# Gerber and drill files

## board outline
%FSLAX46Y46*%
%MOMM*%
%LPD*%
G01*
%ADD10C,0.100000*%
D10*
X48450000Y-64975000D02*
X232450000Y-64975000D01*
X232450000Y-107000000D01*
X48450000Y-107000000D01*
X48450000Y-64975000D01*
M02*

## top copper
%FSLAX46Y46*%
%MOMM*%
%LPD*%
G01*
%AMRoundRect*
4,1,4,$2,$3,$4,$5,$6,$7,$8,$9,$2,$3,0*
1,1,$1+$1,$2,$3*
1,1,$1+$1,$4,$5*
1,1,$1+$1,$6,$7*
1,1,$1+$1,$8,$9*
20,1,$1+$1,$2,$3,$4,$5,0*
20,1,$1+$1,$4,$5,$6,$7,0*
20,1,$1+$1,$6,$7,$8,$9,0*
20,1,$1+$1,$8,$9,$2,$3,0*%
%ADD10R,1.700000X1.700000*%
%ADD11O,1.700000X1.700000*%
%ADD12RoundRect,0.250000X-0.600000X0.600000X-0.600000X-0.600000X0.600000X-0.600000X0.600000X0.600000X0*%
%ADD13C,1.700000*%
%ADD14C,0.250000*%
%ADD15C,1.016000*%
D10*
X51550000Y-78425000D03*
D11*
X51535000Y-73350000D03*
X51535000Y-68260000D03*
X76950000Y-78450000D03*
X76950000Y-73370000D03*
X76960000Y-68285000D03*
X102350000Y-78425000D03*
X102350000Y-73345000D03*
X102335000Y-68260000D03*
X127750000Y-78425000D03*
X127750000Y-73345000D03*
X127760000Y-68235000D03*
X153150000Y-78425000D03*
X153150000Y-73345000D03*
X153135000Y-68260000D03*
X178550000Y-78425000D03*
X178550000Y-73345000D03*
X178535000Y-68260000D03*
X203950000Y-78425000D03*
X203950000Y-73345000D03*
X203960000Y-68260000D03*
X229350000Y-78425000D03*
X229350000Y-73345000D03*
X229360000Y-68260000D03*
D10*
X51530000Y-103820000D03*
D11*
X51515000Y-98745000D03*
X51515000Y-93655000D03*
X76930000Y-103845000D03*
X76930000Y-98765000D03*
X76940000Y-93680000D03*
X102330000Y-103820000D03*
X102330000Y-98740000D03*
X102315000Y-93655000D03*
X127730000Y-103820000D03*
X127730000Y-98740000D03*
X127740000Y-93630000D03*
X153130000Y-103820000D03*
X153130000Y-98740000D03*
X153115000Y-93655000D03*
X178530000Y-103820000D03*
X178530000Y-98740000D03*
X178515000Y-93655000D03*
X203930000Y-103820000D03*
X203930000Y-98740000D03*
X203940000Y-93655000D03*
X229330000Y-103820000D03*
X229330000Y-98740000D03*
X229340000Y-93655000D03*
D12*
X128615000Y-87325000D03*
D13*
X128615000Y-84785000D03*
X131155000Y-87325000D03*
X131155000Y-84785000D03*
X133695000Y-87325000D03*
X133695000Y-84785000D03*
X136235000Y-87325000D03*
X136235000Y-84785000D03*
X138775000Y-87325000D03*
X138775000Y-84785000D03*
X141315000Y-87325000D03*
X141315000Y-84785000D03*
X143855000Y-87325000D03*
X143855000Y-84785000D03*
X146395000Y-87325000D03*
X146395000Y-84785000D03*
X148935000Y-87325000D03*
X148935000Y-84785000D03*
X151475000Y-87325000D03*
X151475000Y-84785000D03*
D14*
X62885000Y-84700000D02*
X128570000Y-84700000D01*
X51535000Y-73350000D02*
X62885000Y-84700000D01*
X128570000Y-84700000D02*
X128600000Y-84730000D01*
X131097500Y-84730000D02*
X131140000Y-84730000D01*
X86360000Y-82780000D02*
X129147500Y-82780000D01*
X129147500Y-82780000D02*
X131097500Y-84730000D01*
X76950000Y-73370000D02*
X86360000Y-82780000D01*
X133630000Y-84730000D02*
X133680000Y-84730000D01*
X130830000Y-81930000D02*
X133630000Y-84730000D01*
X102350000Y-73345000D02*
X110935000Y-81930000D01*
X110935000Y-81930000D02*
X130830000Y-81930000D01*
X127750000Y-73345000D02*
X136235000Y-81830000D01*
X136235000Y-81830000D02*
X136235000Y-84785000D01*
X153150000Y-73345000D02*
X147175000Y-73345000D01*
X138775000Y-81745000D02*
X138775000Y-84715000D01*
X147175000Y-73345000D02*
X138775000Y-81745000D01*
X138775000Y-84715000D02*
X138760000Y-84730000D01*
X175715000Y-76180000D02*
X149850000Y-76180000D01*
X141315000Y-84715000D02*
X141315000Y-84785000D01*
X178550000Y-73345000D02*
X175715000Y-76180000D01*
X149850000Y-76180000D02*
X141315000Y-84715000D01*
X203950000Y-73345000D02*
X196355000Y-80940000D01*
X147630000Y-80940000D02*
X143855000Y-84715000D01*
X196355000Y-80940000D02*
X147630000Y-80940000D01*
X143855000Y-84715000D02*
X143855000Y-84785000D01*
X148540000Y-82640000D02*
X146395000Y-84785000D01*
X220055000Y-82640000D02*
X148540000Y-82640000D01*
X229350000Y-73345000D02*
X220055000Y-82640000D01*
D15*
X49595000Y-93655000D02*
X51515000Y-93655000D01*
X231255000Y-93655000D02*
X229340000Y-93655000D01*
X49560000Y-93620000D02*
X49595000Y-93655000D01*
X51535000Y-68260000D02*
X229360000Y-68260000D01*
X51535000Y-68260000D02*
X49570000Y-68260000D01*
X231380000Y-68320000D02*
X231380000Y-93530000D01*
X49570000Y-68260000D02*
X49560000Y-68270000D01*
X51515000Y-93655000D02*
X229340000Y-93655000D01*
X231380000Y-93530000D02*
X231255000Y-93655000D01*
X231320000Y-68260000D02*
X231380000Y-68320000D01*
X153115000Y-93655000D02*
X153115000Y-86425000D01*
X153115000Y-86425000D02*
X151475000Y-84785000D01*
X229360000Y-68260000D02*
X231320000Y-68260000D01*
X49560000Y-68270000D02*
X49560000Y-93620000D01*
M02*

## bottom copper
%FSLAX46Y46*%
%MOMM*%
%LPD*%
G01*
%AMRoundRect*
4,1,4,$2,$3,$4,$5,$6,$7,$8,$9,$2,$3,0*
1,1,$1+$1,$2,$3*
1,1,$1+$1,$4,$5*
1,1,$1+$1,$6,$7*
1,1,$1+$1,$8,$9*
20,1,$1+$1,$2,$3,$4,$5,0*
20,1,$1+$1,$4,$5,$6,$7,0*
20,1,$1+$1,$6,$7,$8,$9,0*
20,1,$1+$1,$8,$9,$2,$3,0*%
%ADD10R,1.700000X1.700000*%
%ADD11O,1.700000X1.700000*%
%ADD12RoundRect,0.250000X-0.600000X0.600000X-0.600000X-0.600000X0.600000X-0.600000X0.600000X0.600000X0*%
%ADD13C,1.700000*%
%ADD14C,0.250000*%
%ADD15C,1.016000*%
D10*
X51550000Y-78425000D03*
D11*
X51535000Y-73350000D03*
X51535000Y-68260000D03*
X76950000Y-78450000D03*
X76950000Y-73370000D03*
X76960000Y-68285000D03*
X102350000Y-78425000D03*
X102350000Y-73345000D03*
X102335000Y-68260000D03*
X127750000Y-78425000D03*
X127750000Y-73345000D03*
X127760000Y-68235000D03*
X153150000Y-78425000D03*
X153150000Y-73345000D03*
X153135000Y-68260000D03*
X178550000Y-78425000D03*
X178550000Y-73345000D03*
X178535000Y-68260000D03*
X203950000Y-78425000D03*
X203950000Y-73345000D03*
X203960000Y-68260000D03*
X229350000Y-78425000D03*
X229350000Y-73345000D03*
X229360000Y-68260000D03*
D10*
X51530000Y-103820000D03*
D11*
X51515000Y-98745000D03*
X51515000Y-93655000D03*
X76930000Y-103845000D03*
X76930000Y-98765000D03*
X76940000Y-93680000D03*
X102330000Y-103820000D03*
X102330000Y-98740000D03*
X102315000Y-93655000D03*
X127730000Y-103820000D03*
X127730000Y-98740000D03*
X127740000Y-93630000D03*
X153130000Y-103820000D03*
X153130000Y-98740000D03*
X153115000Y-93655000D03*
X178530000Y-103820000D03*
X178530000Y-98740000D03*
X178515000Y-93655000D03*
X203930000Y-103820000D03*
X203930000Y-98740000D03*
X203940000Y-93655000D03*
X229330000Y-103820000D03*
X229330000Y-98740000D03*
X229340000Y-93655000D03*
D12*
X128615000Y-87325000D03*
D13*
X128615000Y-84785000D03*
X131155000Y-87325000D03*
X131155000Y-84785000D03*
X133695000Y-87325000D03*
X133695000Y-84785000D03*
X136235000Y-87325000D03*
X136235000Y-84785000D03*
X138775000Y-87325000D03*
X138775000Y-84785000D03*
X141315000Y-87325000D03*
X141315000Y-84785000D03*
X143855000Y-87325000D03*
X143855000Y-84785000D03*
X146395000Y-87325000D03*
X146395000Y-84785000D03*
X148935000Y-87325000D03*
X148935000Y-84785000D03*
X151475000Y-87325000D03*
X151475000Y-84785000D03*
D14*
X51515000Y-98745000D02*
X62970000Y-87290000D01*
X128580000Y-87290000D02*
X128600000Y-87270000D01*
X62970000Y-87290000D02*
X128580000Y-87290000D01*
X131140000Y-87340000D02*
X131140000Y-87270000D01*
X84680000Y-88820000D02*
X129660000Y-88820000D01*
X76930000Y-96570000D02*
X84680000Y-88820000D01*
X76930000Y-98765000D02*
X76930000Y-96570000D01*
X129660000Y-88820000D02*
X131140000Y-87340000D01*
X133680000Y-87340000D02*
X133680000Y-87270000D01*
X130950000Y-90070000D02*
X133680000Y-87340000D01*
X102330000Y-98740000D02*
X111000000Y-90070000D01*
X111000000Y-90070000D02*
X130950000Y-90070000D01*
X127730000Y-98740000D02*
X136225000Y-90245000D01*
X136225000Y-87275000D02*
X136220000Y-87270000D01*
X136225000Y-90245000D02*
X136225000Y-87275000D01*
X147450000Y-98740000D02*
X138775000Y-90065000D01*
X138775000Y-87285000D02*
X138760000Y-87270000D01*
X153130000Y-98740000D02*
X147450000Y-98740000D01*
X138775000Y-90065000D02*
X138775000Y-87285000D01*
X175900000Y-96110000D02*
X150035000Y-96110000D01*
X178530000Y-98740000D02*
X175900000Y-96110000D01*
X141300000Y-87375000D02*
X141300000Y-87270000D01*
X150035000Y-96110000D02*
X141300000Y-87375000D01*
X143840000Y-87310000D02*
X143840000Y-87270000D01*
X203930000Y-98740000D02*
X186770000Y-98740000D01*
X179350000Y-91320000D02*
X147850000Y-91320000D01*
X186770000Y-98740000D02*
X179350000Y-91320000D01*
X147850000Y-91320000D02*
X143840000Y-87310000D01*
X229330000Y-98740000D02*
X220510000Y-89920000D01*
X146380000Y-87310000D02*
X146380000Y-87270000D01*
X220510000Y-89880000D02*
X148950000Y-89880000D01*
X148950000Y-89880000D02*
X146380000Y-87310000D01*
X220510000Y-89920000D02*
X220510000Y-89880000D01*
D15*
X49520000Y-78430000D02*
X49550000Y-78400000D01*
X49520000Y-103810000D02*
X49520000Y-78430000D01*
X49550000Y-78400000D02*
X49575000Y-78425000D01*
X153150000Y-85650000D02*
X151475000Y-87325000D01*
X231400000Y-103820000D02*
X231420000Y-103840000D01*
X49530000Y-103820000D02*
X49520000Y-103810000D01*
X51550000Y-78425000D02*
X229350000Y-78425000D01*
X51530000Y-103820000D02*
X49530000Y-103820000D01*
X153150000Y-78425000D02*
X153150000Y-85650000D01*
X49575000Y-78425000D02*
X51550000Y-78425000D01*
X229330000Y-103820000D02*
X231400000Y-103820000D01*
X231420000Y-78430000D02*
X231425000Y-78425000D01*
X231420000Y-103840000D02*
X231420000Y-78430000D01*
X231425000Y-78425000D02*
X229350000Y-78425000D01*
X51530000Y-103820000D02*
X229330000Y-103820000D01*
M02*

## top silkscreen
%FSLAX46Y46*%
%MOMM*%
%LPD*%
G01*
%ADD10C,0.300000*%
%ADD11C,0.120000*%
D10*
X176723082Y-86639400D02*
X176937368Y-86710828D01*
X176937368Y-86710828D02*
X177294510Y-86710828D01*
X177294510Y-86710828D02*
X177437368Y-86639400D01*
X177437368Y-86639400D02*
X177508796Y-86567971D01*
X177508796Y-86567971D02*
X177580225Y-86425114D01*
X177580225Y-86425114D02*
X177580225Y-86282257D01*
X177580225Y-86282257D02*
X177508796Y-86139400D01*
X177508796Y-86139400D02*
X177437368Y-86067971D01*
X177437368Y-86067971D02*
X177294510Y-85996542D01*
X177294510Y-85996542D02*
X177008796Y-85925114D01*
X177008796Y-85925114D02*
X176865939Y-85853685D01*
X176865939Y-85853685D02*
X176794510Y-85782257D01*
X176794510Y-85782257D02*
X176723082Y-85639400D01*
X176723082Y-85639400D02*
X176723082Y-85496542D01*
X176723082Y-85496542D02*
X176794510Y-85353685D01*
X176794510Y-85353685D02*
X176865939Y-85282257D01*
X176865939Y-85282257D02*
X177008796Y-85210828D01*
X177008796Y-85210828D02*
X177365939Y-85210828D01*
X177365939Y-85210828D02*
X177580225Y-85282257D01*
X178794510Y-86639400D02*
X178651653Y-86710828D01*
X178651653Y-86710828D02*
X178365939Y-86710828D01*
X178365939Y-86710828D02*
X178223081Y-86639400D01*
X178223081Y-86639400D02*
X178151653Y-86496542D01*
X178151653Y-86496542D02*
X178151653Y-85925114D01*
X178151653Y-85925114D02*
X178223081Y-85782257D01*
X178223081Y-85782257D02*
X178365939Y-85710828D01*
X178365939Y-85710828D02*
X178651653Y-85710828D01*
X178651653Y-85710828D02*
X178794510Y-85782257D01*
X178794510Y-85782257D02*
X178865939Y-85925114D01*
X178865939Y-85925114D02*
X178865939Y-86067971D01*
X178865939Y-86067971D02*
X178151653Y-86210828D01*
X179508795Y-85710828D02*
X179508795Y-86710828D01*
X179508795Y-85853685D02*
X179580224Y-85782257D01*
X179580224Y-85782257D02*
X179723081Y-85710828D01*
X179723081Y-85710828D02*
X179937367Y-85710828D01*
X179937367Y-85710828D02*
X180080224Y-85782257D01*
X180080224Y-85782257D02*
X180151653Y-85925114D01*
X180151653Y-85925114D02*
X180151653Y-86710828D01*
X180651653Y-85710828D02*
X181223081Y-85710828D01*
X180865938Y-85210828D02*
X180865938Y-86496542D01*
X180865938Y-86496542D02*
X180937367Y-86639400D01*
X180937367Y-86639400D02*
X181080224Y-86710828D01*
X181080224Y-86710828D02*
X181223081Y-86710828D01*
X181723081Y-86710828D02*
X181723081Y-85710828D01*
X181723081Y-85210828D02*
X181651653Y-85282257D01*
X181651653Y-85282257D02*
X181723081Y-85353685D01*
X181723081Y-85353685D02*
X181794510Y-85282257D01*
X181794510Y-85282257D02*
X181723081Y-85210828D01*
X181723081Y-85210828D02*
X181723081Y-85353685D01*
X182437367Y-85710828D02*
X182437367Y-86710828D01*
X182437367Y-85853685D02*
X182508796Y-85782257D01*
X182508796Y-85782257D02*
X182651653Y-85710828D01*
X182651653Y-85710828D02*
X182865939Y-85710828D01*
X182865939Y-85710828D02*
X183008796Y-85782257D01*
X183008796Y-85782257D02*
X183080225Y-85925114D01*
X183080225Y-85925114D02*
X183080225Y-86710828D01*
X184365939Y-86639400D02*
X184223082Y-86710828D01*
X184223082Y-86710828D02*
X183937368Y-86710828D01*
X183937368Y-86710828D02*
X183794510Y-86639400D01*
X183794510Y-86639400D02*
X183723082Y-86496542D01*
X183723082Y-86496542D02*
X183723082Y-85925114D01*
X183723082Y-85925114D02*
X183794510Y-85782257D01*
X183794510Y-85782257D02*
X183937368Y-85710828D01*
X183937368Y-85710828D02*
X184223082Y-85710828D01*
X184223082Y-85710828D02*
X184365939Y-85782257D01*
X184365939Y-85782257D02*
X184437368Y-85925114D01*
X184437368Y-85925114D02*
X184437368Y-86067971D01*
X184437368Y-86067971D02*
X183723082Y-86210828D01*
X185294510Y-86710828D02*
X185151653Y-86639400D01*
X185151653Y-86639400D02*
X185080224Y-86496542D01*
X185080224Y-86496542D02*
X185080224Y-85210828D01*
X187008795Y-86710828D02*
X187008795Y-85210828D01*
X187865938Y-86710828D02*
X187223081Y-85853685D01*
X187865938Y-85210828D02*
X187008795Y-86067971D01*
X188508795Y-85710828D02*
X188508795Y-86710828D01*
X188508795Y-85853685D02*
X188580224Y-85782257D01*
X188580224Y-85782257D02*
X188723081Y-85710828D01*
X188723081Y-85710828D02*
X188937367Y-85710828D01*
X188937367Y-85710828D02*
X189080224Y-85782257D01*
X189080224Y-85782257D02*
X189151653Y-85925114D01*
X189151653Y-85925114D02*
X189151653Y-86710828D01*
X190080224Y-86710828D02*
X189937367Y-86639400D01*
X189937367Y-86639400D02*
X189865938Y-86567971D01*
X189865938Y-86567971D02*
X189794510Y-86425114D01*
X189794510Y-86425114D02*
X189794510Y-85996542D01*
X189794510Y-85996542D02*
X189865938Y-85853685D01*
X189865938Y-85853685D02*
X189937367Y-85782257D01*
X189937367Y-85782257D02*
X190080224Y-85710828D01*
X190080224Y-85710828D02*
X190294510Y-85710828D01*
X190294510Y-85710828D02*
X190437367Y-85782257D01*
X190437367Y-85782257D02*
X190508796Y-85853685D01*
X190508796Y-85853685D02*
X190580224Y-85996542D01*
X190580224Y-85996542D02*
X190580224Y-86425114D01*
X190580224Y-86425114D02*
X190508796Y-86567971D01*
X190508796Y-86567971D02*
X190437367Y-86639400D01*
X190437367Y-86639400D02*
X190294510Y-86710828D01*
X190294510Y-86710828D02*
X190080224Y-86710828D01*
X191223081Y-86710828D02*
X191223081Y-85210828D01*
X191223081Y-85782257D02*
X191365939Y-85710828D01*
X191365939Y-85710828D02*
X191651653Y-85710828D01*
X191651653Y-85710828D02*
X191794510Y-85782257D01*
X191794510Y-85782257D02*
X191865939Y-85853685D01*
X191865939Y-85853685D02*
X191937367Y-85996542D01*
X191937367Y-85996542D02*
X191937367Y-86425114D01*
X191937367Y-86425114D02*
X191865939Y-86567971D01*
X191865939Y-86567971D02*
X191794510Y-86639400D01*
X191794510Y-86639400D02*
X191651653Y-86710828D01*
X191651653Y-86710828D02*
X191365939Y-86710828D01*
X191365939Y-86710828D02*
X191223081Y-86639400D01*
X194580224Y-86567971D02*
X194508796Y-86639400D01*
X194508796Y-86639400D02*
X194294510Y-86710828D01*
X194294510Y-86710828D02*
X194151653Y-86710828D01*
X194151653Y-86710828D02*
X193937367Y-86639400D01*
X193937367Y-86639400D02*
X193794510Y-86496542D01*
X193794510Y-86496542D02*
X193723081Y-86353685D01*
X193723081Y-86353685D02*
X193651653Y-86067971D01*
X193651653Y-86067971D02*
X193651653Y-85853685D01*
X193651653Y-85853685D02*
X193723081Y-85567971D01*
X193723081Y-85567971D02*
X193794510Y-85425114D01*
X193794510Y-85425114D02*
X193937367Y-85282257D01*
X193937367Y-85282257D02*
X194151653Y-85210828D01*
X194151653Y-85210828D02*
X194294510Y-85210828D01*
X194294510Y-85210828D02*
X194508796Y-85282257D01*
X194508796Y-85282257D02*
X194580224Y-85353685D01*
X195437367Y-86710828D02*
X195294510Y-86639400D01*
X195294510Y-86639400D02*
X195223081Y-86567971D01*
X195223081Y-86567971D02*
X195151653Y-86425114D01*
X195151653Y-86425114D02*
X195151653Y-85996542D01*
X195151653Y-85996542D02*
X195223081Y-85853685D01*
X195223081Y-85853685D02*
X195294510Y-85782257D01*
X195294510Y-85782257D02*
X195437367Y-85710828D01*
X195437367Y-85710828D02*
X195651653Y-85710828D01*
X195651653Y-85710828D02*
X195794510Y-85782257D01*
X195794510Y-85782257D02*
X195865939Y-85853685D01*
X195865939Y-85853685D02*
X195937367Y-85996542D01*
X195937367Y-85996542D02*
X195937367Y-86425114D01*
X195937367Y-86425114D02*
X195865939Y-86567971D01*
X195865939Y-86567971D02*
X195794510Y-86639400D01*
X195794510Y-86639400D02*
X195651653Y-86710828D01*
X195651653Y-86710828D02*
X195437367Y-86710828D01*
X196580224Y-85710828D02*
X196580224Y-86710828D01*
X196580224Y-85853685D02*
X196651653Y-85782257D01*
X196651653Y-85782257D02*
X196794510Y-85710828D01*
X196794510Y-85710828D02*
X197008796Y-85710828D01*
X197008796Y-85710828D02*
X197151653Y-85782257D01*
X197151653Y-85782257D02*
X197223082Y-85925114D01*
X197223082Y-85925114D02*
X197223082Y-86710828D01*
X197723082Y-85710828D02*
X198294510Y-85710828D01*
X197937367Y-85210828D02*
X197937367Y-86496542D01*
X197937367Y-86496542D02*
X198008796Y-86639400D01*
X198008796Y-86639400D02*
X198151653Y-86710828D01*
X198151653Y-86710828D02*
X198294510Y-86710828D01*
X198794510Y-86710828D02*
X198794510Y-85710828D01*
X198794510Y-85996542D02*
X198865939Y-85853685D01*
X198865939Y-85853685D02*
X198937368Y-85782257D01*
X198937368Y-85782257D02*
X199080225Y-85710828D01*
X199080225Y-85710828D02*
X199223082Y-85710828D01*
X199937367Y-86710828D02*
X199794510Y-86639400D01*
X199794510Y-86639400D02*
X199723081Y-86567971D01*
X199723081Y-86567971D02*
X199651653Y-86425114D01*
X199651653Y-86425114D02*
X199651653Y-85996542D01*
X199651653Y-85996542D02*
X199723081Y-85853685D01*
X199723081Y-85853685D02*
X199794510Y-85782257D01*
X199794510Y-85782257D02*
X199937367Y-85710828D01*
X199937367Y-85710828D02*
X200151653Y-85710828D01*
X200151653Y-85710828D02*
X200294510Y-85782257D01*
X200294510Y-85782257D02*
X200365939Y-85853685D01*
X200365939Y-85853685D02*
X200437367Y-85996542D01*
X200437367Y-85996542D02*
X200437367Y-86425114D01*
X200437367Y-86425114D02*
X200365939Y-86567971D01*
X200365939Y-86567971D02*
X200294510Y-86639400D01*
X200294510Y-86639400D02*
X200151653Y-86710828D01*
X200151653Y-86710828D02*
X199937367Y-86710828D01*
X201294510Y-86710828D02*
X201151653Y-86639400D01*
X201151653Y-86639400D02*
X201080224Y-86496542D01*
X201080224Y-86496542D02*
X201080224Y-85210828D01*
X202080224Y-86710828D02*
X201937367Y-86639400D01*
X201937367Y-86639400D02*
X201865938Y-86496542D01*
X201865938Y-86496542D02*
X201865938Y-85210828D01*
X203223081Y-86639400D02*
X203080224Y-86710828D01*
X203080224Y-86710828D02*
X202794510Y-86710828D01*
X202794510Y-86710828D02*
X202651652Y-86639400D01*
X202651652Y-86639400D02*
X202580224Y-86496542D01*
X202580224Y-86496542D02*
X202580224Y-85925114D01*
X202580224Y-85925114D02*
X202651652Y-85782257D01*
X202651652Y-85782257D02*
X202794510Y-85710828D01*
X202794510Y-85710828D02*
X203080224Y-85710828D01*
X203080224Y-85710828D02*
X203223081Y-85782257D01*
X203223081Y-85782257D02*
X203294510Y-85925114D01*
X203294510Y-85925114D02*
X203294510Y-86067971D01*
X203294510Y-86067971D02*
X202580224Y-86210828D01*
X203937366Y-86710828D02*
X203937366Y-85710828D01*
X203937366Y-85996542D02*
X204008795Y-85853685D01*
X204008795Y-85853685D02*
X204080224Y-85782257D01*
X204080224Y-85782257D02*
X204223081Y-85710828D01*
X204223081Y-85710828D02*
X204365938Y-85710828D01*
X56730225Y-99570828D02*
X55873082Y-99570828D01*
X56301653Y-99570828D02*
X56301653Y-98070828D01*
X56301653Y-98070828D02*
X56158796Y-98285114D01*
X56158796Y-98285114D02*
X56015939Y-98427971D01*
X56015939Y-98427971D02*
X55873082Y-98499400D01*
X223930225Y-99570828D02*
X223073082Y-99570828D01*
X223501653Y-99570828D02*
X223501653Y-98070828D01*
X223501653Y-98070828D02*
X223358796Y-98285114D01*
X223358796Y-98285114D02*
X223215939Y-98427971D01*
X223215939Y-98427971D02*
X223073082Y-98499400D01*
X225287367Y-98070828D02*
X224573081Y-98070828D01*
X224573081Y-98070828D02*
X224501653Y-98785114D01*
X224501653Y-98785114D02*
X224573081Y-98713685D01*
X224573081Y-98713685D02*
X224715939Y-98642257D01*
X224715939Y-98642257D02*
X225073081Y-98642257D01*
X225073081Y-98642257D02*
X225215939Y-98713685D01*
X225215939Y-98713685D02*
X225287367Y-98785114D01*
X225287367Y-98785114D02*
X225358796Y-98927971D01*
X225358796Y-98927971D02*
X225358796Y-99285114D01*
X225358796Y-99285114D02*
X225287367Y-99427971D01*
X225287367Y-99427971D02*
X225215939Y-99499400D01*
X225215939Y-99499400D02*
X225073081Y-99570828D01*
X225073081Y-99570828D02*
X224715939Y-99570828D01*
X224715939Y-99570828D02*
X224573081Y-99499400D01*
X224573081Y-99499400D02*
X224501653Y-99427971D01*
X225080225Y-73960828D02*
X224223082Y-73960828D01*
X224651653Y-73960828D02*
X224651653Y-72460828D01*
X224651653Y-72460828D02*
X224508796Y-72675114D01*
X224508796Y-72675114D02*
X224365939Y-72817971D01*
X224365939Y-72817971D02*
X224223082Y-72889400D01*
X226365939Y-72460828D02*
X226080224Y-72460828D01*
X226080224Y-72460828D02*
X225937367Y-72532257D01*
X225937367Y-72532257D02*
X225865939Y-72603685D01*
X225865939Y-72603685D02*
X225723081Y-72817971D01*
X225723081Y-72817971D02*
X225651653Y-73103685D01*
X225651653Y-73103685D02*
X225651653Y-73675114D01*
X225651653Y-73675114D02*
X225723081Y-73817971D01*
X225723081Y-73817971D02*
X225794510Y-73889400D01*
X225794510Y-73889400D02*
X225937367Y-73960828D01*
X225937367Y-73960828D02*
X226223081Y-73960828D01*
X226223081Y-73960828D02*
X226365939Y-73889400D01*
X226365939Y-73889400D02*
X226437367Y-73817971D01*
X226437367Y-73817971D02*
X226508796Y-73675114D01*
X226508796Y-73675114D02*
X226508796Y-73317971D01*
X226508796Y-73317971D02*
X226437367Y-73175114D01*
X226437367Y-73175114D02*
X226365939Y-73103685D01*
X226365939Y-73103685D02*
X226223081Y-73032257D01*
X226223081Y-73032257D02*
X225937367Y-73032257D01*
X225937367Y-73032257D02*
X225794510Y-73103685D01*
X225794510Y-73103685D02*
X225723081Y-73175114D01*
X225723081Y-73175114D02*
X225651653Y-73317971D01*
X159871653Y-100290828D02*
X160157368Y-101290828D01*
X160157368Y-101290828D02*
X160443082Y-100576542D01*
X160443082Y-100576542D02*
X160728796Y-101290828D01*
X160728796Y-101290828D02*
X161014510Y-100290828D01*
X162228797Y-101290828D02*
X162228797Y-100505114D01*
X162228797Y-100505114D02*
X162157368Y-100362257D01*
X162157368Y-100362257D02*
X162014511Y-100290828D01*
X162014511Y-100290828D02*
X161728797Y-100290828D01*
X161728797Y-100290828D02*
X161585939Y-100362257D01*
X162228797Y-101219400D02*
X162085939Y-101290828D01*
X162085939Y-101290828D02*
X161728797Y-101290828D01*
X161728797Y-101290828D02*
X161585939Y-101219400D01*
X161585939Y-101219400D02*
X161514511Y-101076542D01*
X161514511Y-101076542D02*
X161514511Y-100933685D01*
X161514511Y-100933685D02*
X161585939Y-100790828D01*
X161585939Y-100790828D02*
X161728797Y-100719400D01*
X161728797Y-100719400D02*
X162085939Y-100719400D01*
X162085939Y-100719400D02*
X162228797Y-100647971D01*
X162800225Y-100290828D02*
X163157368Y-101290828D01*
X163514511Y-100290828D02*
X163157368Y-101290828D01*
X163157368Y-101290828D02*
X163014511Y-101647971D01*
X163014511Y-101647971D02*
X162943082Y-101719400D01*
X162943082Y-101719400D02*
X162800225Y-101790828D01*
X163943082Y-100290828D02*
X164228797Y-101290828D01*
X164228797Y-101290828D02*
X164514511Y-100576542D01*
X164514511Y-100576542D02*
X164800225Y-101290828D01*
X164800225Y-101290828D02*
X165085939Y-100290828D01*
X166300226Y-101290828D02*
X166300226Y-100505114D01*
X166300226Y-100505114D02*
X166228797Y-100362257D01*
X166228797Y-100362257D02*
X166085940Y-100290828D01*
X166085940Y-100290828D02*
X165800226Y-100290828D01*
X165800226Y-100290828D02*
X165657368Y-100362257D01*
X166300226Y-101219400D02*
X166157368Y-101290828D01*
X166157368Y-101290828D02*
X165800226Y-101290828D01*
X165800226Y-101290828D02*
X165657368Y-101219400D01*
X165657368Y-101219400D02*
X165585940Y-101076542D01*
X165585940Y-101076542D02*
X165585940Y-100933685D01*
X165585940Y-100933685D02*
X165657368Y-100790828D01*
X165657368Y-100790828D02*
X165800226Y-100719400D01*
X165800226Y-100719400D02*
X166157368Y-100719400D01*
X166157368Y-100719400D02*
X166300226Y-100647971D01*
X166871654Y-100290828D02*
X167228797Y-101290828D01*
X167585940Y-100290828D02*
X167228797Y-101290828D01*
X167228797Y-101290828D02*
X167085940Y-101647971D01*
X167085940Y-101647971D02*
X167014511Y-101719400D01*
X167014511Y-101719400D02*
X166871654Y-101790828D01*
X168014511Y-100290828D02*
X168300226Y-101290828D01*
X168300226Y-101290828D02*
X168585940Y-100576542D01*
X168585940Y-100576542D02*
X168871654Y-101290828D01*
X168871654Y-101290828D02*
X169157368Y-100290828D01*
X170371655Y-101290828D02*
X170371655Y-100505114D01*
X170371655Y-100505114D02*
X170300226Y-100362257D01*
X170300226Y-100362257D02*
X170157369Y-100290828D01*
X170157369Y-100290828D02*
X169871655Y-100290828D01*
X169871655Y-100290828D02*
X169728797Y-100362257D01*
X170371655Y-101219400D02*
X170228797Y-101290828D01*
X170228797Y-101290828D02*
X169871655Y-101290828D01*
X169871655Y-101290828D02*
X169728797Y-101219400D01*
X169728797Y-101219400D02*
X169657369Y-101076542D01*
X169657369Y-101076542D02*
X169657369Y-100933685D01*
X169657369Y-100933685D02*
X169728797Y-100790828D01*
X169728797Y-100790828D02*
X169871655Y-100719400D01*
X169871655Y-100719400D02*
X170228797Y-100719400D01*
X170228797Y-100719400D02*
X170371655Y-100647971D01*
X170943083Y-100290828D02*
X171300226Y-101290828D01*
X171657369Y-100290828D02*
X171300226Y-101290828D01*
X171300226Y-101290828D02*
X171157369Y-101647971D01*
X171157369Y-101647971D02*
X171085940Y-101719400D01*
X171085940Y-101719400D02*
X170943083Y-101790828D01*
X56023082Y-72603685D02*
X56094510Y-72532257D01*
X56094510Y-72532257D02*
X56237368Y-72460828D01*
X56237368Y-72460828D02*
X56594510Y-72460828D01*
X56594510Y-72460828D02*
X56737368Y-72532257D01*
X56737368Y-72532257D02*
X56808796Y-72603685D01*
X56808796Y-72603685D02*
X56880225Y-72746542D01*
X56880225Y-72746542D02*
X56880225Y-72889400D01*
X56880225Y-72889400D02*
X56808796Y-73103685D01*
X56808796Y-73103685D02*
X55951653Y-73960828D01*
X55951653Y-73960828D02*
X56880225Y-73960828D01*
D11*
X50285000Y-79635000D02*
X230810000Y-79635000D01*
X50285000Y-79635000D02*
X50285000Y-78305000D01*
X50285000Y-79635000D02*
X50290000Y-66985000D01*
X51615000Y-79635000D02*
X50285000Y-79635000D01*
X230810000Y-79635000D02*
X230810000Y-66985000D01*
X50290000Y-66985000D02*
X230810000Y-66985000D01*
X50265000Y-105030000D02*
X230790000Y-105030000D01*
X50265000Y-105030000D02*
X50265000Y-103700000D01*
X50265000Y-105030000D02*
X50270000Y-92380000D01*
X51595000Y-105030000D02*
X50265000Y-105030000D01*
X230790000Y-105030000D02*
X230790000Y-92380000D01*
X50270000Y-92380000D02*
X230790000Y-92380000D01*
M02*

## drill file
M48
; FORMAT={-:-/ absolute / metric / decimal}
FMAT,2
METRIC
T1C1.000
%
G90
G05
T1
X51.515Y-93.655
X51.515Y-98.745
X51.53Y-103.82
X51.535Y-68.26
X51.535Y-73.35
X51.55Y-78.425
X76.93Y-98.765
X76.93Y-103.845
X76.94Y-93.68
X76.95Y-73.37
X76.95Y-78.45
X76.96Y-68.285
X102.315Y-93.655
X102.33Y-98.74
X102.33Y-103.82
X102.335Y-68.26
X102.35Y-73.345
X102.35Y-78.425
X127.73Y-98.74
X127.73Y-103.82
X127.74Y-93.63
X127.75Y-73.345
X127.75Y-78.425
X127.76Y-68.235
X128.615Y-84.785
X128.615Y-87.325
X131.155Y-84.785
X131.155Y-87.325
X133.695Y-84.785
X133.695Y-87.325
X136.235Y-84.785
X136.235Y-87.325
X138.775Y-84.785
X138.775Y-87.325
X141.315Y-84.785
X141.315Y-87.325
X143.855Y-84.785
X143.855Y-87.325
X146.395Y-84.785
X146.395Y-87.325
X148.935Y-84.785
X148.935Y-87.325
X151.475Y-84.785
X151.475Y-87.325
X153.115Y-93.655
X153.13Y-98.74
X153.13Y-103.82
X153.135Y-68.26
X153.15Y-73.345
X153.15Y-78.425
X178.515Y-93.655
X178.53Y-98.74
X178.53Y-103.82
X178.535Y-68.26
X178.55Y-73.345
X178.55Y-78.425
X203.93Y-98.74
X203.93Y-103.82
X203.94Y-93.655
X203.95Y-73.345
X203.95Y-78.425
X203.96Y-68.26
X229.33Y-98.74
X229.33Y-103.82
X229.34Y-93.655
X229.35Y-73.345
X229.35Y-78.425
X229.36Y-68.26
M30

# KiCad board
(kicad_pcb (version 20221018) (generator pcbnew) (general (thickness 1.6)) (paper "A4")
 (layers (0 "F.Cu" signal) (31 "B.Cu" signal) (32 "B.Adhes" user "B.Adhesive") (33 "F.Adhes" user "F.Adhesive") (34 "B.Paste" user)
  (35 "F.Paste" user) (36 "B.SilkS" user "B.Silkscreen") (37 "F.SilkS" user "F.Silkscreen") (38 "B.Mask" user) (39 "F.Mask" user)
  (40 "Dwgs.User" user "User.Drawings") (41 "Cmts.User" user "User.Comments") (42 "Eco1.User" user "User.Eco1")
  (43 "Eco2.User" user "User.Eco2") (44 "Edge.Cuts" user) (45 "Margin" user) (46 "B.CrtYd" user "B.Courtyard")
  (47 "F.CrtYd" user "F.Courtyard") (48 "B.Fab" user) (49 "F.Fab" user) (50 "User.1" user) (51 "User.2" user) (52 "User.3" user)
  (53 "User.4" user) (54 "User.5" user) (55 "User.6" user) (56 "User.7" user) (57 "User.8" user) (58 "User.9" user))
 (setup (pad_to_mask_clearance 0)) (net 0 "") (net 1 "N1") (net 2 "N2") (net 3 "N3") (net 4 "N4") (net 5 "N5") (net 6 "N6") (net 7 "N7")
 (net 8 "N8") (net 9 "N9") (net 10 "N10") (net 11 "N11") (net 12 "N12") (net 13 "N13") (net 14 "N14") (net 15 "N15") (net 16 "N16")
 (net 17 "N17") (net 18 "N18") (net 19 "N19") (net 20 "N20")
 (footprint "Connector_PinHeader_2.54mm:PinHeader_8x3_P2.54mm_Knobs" (layer "F.Cu") (at 49.01 75.885 90)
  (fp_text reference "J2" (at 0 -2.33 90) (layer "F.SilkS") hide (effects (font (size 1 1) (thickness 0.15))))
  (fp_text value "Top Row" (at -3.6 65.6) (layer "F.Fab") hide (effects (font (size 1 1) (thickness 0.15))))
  (fp_line (start -3.75 1.275) (end -3.75 181.8) (stroke (width 0.12) (type solid)) (layer "F.SilkS"))
  (fp_line (start -3.75 1.275) (end -2.42 1.275) (stroke (width 0.12) (type solid)) (layer "F.SilkS"))
  (fp_line (start -3.75 1.275) (end 8.9 1.28) (stroke (width 0.12) (type solid)) (layer "F.SilkS"))
  (fp_line (start -3.75 2.605) (end -3.75 1.275) (stroke (width 0.12) (type solid)) (layer "F.SilkS"))
  (fp_line (start -3.75 181.8) (end 8.9 181.8) (stroke (width 0.12) (type solid)) (layer "F.SilkS"))
  (fp_line (start 8.9 1.28) (end 8.9 181.8) (stroke (width 0.12) (type solid)) (layer "F.SilkS"))
  (pad "1" thru_hole rect (at -2.54 2.54 180) (size 1.7 1.7) (drill 1) (layers "*.Cu" "*.Mask") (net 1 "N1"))
  (pad "2" thru_hole oval (at 2.535 2.525 180) (size 1.7 1.7) (drill 1) (layers "*.Cu" "*.Mask") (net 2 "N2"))
  (pad "3" thru_hole oval (at 7.625 2.525 180) (size 1.7 1.7) (drill 1) (layers "*.Cu" "*.Mask") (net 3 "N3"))
  (pad "4" thru_hole oval (at -2.565 27.94 180) (size 1.7 1.7) (drill 1) (layers "*.Cu" "*.Mask") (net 1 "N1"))
  (pad "5" thru_hole oval (at 2.515 27.94 180) (size 1.7 1.7) (drill 1) (layers "*.Cu" "*.Mask") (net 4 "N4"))
  (pad "6" thru_hole oval (at 7.6 27.95 180) (size 1.7 1.7) (drill 1) (layers "*.Cu" "*.Mask") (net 3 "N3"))
  (pad "7" thru_hole oval (at -2.54 53.34 180) (size 1.7 1.7) (drill 1) (layers "*.Cu" "*.Mask") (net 1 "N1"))
  (pad "8" thru_hole oval (at 2.54 53.34 180) (size 1.7 1.7) (drill 1) (layers "*.Cu" "*.Mask") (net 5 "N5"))
  (pad "9" thru_hole oval (at 7.625 53.325 180) (size 1.7 1.7) (drill 1) (layers "*.Cu" "*.Mask") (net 3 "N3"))
  (pad "10" thru_hole oval (at -2.54 78.74 180) (size 1.7 1.7) (drill 1) (layers "*.Cu" "*.Mask") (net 1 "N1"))
  (pad "11" thru_hole oval (at 2.54 78.74 180) (size 1.7 1.7) (drill 1) (layers "*.Cu" "*.Mask") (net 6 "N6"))
  (pad "12" thru_hole oval (at 7.65 78.75 180) (size 1.7 1.7) (drill 1) (layers "*.Cu" "*.Mask") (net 3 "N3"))
  (pad "13" thru_hole oval (at -2.54 104.14 180) (size 1.7 1.7) (drill 1) (layers "*.Cu" "*.Mask") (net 1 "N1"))
  (pad "14" thru_hole oval (at 2.54 104.14 180) (size 1.7 1.7) (drill 1) (layers "*.Cu" "*.Mask") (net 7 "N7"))
  (pad "15" thru_hole oval (at 7.625 104.125 180) (size 1.7 1.7) (drill 1) (layers "*.Cu" "*.Mask") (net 3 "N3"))
  (pad "16" thru_hole oval (at -2.54 129.54 180) (size 1.7 1.7) (drill 1) (layers "*.Cu" "*.Mask") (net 1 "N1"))
  (pad "17" thru_hole oval (at 2.54 129.54 180) (size 1.7 1.7) (drill 1) (layers "*.Cu" "*.Mask") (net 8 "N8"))
  (pad "18" thru_hole oval (at 7.625 129.525 180) (size 1.7 1.7) (drill 1) (layers "*.Cu" "*.Mask") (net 3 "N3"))
  (pad "19" thru_hole oval (at -2.54 154.94 180) (size 1.7 1.7) (drill 1) (layers "*.Cu" "*.Mask") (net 1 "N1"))
  (pad "20" thru_hole oval (at 2.54 154.94 180) (size 1.7 1.7) (drill 1) (layers "*.Cu" "*.Mask") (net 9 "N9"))
  (pad "21" thru_hole oval (at 7.625 154.95 180) (size 1.7 1.7) (drill 1) (layers "*.Cu" "*.Mask") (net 3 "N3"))
  (pad "22" thru_hole oval (at -2.54 180.34 180) (size 1.7 1.7) (drill 1) (layers "*.Cu" "*.Mask") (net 1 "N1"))
  (pad "23" thru_hole oval (at 2.54 180.34 180) (size 1.7 1.7) (drill 1) (layers "*.Cu" "*.Mask") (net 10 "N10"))
  (pad "24" thru_hole oval (at 7.625 180.35 180) (size 1.7 1.7) (drill 1) (layers "*.Cu" "*.Mask") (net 3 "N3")))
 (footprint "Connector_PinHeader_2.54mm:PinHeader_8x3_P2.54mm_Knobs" (layer "F.Cu") (at 48.99 101.28 90)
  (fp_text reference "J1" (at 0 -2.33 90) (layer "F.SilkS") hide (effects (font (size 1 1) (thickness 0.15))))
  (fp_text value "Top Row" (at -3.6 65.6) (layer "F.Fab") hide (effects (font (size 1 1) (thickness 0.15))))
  (fp_line (start -3.75 1.275) (end -3.75 181.8) (stroke (width 0.12) (type solid)) (layer "F.SilkS"))
  (fp_line (start -3.75 1.275) (end -2.42 1.275) (stroke (width 0.12) (type solid)) (layer "F.SilkS"))
  (fp_line (start -3.75 1.275) (end 8.9 1.28) (stroke (width 0.12) (type solid)) (layer "F.SilkS"))
  (fp_line (start -3.75 2.605) (end -3.75 1.275) (stroke (width 0.12) (type solid)) (layer "F.SilkS"))
  (fp_line (start -3.75 181.8) (end 8.9 181.8) (stroke (width 0.12) (type solid)) (layer "F.SilkS"))
  (fp_line (start 8.9 1.28) (end 8.9 181.8) (stroke (width 0.12) (type solid)) (layer "F.SilkS"))
  (pad "1" thru_hole rect (at -2.54 2.54 180) (size 1.7 1.7) (drill 1) (layers "*.Cu" "*.Mask") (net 1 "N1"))
  (pad "2" thru_hole oval (at 2.535 2.525 180) (size 1.7 1.7) (drill 1) (layers "*.Cu" "*.Mask") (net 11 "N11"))
  (pad "3" thru_hole oval (at 7.625 2.525 180) (size 1.7 1.7) (drill 1) (layers "*.Cu" "*.Mask") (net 3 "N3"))
  (pad "4" thru_hole oval (at -2.565 27.94 180) (size 1.7 1.7) (drill 1) (layers "*.Cu" "*.Mask") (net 1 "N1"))
  (pad "5" thru_hole oval (at 2.515 27.94 180) (size 1.7 1.7) (drill 1) (layers "*.Cu" "*.Mask") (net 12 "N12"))
  (pad "6" thru_hole oval (at 7.6 27.95 180) (size 1.7 1.7) (drill 1) (layers "*.Cu" "*.Mask") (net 3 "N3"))
  (pad "7" thru_hole oval (at -2.54 53.34 180) (size 1.7 1.7) (drill 1) (layers "*.Cu" "*.Mask") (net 1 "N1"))
  (pad "8" thru_hole oval (at 2.54 53.34 180) (size 1.7 1.7) (drill 1) (layers "*.Cu" "*.Mask") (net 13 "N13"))
  (pad "9" thru_hole oval (at 7.625 53.325 180) (size 1.7 1.7) (drill 1) (layers "*.Cu" "*.Mask") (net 3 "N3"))
  (pad "10" thru_hole oval (at -2.54 78.74 180) (size 1.7 1.7) (drill 1) (layers "*.Cu" "*.Mask") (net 1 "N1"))
  (pad "11" thru_hole oval (at 2.54 78.74 180) (size 1.7 1.7) (drill 1) (layers "*.Cu" "*.Mask") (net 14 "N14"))
  (pad "12" thru_hole oval (at 7.65 78.75 180) (size 1.7 1.7) (drill 1) (layers "*.Cu" "*.Mask") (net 3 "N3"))
  (pad "13" thru_hole oval (at -2.54 104.14 180) (size 1.7 1.7) (drill 1) (layers "*.Cu" "*.Mask") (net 1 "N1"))
  (pad "14" thru_hole oval (at 2.54 104.14 180) (size 1.7 1.7) (drill 1) (layers "*.Cu" "*.Mask") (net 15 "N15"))
  (pad "15" thru_hole oval (at 7.625 104.125 180) (size 1.7 1.7) (drill 1) (layers "*.Cu" "*.Mask") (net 3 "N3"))
  (pad "16" thru_hole oval (at -2.54 129.54 180) (size 1.7 1.7) (drill 1) (layers "*.Cu" "*.Mask") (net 1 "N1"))
  (pad "17" thru_hole oval (at 2.54 129.54 180) (size 1.7 1.7) (drill 1) (layers "*.Cu" "*.Mask") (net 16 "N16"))
  (pad "18" thru_hole oval (at 7.625 129.525 180) (size 1.7 1.7) (drill 1) (layers "*.Cu" "*.Mask") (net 3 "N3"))
  (pad "19" thru_hole oval (at -2.54 154.94 180) (size 1.7 1.7) (drill 1) (layers "*.Cu" "*.Mask") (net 1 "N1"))
  (pad "20" thru_hole oval (at 2.54 154.94 180) (size 1.7 1.7) (drill 1) (layers "*.Cu" "*.Mask") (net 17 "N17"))
  (pad "21" thru_hole oval (at 7.625 154.95 180) (size 1.7 1.7) (drill 1) (layers "*.Cu" "*.Mask") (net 3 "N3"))
  (pad "22" thru_hole oval (at -2.54 180.34 180) (size 1.7 1.7) (drill 1) (layers "*.Cu" "*.Mask") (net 1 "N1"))
  (pad "23" thru_hole oval (at 2.54 180.34 180) (size 1.7 1.7) (drill 1) (layers "*.Cu" "*.Mask") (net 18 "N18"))
  (pad "24" thru_hole oval (at 7.625 180.35 180) (size 1.7 1.7) (drill 1) (layers "*.Cu" "*.Mask") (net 3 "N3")))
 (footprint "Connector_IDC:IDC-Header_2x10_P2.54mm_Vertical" (layer "B.Cu") (at 128.615 84.785 -90)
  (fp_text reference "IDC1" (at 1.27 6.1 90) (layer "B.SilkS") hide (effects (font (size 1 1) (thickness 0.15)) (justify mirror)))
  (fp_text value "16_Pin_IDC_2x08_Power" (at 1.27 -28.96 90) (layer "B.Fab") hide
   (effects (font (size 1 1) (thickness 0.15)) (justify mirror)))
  (pad "1" thru_hole roundrect (at 2.54 0 270) (size 1.7 1.7) (drill 1) (layers "*.Cu" "*.Mask") (roundrect_rratio 0.1470588235)
   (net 11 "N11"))
  (pad "2" thru_hole circle (at 0 0 270) (size 1.7 1.7) (drill 1) (layers "*.Cu" "*.Mask") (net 2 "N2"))
  (pad "3" thru_hole circle (at 2.54 -2.54 270) (size 1.7 1.7) (drill 1) (layers "*.Cu" "*.Mask") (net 12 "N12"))
  (pad "4" thru_hole circle (at 0 -2.54 270) (size 1.7 1.7) (drill 1) (layers "*.Cu" "*.Mask") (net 4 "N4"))
  (pad "5" thru_hole circle (at 2.54 -5.08 270) (size 1.7 1.7) (drill 1) (layers "*.Cu" "*.Mask") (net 13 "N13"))
  (pad "6" thru_hole circle (at 0 -5.08 270) (size 1.7 1.7) (drill 1) (layers "*.Cu" "*.Mask") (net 5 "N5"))
  (pad "7" thru_hole circle (at 2.54 -7.62 270) (size 1.7 1.7) (drill 1) (layers "*.Cu" "*.Mask") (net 14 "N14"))
  (pad "8" thru_hole circle (at 0 -7.62 270) (size 1.7 1.7) (drill 1) (layers "*.Cu" "*.Mask") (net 6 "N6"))
  (pad "9" thru_hole circle (at 2.54 -10.16 270) (size 1.7 1.7) (drill 1) (layers "*.Cu" "*.Mask") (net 15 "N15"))
  (pad "10" thru_hole circle (at 0 -10.16 270) (size 1.7 1.7) (drill 1) (layers "*.Cu" "*.Mask") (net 7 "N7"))
  (pad "11" thru_hole circle (at 2.54 -12.7 270) (size 1.7 1.7) (drill 1) (layers "*.Cu" "*.Mask") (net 16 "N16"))
  (pad "12" thru_hole circle (at 0 -12.7 270) (size 1.7 1.7) (drill 1) (layers "*.Cu" "*.Mask") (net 8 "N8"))
  (pad "13" thru_hole circle (at 2.54 -15.24 270) (size 1.7 1.7) (drill 1) (layers "*.Cu" "*.Mask") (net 17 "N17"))
  (pad "14" thru_hole circle (at 0 -15.24 270) (size 1.7 1.7) (drill 1) (layers "*.Cu" "*.Mask") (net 9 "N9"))
  (pad "15" thru_hole circle (at 2.54 -17.78 270) (size 1.7 1.7) (drill 1) (layers "*.Cu" "*.Mask") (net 18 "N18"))
  (pad "16" thru_hole circle (at 0 -17.78 270) (size 1.7 1.7) (drill 1) (layers "*.Cu" "*.Mask") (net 10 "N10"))
  (pad "17" thru_hole circle (at 2.54 -20.32 270) (size 1.7 1.7) (drill 1) (layers "*.Cu" "*.Mask") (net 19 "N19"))
  (pad "18" thru_hole circle (at 0 -20.32 270) (size 1.7 1.7) (drill 1) (layers "*.Cu" "*.Mask") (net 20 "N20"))
  (pad "19" thru_hole circle (at 2.54 -22.86 270) (size 1.7 1.7) (drill 1) (layers "*.Cu" "*.Mask") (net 1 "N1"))
  (pad "20" thru_hole circle (at 0 -22.86 270) (size 1.7 1.7) (drill 1) (layers "*.Cu" "*.Mask") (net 3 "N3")))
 (gr_rect (start 48.45 64.975) (end 232.45 107) (stroke (width 0.1) (type default)) (fill none) (layer "Edge.Cuts"))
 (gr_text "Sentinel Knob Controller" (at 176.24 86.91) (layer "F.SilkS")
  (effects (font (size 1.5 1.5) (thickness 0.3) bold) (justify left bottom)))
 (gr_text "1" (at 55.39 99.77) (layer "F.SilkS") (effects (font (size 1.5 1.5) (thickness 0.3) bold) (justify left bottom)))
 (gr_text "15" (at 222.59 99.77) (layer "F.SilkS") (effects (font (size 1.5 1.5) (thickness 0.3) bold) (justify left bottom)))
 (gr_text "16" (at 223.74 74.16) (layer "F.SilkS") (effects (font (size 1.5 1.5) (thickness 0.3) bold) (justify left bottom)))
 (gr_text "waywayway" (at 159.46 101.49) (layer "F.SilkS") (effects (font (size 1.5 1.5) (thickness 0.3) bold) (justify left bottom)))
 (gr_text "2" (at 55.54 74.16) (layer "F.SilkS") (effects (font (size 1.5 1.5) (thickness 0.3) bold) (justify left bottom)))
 (segment (start 51.515 98.745) (end 62.97 87.29) (width 0.25) (layer "B.Cu") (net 11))
 (segment (start 128.58 87.29) (end 128.6 87.27) (width 0.25) (layer "B.Cu") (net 11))
 (segment (start 62.97 87.29) (end 128.58 87.29) (width 0.25) (layer "B.Cu") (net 11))
 (segment (start 62.885 84.7) (end 128.57 84.7) (width 0.25) (layer "F.Cu") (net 2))
 (segment (start 51.535 73.35) (end 62.885 84.7) (width 0.25) (layer "F.Cu") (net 2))
 (segment (start 128.57 84.7) (end 128.6 84.73) (width 0.25) (layer "F.Cu") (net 2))
 (segment (start 131.14 87.34) (end 131.14 87.27) (width 0.25) (layer "B.Cu") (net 12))
 (segment (start 84.68 88.82) (end 129.66 88.82) (width 0.25) (layer "B.Cu") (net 12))
 (segment (start 76.93 96.57) (end 84.68 88.82) (width 0.25) (layer "B.Cu") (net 12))
 (segment (start 76.93 98.765) (end 76.93 96.57) (width 0.25) (layer "B.Cu") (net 12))
 (segment (start 129.66 88.82) (end 131.14 87.34) (width 0.25) (layer "B.Cu") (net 12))
 (segment (start 131.0975 84.73) (end 131.14 84.73) (width 0.25) (layer "F.Cu") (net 4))
 (segment (start 86.36 82.78) (end 129.1475 82.78) (width 0.25) (layer "F.Cu") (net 4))
 (segment (start 129.1475 82.78) (end 131.0975 84.73) (width 0.25) (layer "F.Cu") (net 4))
 (segment (start 76.95 73.37) (end 86.36 82.78) (width 0.25) (layer "F.Cu") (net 4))
 (segment (start 133.68 87.34) (end 133.68 87.27) (width 0.25) (layer "B.Cu") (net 13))
 (segment (start 130.95 90.07) (end 133.68 87.34) (width 0.25) (layer "B.Cu") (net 13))
 (segment (start 102.33 98.74) (end 111 90.07) (width 0.25) (layer "B.Cu") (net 13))
 (segment (start 111 90.07) (end 130.95 90.07) (width 0.25) (layer "B.Cu") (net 13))
 (segment (start 133.63 84.73) (end 133.68 84.73) (width 0.25) (layer "F.Cu") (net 5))
 (segment (start 130.83 81.93) (end 133.63 84.73) (width 0.25) (layer "F.Cu") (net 5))
 (segment (start 102.35 73.345) (end 110.935 81.93) (width 0.25) (layer "F.Cu") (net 5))
 (segment (start 110.935 81.93) (end 130.83 81.93) (width 0.25) (layer "F.Cu") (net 5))
 (segment (start 127.73 98.74) (end 136.225 90.245) (width 0.25) (layer "B.Cu") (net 14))
 (segment (start 136.225 87.275) (end 136.22 87.27) (width 0.25) (layer "B.Cu") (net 14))
 (segment (start 136.225 90.245) (end 136.225 87.275) (width 0.25) (layer "B.Cu") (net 14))
 (segment (start 127.75 73.345) (end 136.235 81.83) (width 0.25) (layer "F.Cu") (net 6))
 (segment (start 136.235 81.83) (end 136.235 84.785) (width 0.25) (layer "F.Cu") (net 6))
 (segment (start 147.45 98.74) (end 138.775 90.065) (width 0.25) (layer "B.Cu") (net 15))
 (segment (start 138.775 87.285) (end 138.76 87.27) (width 0.25) (layer "B.Cu") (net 15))
 (segment (start 153.13 98.74) (end 147.45 98.74) (width 0.25) (layer "B.Cu") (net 15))
 (segment (start 138.775 90.065) (end 138.775 87.285) (width 0.25) (layer "B.Cu") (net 15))
 (segment (start 153.15 73.345) (end 147.175 73.345) (width 0.25) (layer "F.Cu") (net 7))
 (segment (start 138.775 81.745) (end 138.775 84.715) (width 0.25) (layer "F.Cu") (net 7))
 (segment (start 147.175 73.345) (end 138.775 81.745) (width 0.25) (layer "F.Cu") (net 7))
 (segment (start 138.775 84.715) (end 138.76 84.73) (width 0.25) (layer "F.Cu") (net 7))
 (segment (start 175.9 96.11) (end 150.035 96.11) (width 0.25) (layer "B.Cu") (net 16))
 (segment (start 178.53 98.74) (end 175.9 96.11) (width 0.25) (layer "B.Cu") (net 16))
 (segment (start 141.3 87.375) (end 141.3 87.27) (width 0.25) (layer "B.Cu") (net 16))
 (segment (start 150.035 96.11) (end 141.3 87.375) (width 0.25) (layer "B.Cu") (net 16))
 (segment (start 175.715 76.18) (end 149.85 76.18) (width 0.25) (layer "F.Cu") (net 8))
 (segment (start 141.315 84.715) (end 141.315 84.785) (width 0.25) (layer "F.Cu") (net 8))
 (segment (start 178.55 73.345) (end 175.715 76.18) (width 0.25) (layer "F.Cu") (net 8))
 (segment (start 149.85 76.18) (end 141.315 84.715) (width 0.25) (layer "F.Cu") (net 8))
 (segment (start 143.84 87.31) (end 143.84 87.27) (width 0.25) (layer "B.Cu") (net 17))
 (segment (start 203.93 98.74) (end 186.77 98.74) (width 0.25) (layer "B.Cu") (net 17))
 (segment (start 179.35 91.32) (end 147.85 91.32) (width 0.25) (layer "B.Cu") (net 17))
 (segment (start 186.77 98.74) (end 179.35 91.32) (width 0.25) (layer "B.Cu") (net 17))
 (segment (start 147.85 91.32) (end 143.84 87.31) (width 0.25) (layer "B.Cu") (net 17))
 (segment (start 203.95 73.345) (end 196.355 80.94) (width 0.25) (layer "F.Cu") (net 9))
 (segment (start 147.63 80.94) (end 143.855 84.715) (width 0.25) (layer "F.Cu") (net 9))
 (segment (start 196.355 80.94) (end 147.63 80.94) (width 0.25) (layer "F.Cu") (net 9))
 (segment (start 143.855 84.715) (end 143.855 84.785) (width 0.25) (layer "F.Cu") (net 9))
 (segment (start 229.33 98.74) (end 220.51 89.92) (width 0.25) (layer "B.Cu") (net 18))
 (segment (start 146.38 87.31) (end 146.38 87.27) (width 0.25) (layer "B.Cu") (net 18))
 (segment (start 220.51 89.88) (end 148.95 89.88) (width 0.25) (layer "B.Cu") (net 18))
 (segment (start 148.95 89.88) (end 146.38 87.31) (width 0.25) (layer "B.Cu") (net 18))
 (segment (start 220.51 89.92) (end 220.51 89.88) (width 0.25) (layer "B.Cu") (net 18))
 (segment (start 148.54 82.64) (end 146.395 84.785) (width 0.25) (layer "F.Cu") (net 10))
 (segment (start 220.055 82.64) (end 148.54 82.64) (width 0.25) (layer "F.Cu") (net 10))
 (segment (start 229.35 73.345) (end 220.055 82.64) (width 0.25) (layer "F.Cu") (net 10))
 (segment (start 49.52 78.43) (end 49.55 78.4) (width 1.016) (layer "B.Cu") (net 1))
 (segment (start 49.52 103.81) (end 49.52 78.43) (width 1.016) (layer "B.Cu") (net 1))
 (segment (start 49.55 78.4) (end 49.575 78.425) (width 1.016) (layer "B.Cu") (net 1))
 (segment (start 153.15 85.65) (end 151.475 87.325) (width 1.016) (layer "B.Cu") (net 1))
 (segment (start 231.4 103.82) (end 231.42 103.84) (width 1.016) (layer "B.Cu") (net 1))
 (segment (start 49.53 103.82) (end 49.52 103.81) (width 1.016) (layer "B.Cu") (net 1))
 (segment (start 51.55 78.425) (end 229.35 78.425) (width 1.016) (layer "B.Cu") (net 1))
 (segment (start 51.53 103.82) (end 49.53 103.82) (width 1.016) (layer "B.Cu") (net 1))
 (segment (start 153.15 78.425) (end 153.15 85.65) (width 1.016) (layer "B.Cu") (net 1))
 (segment (start 49.575 78.425) (end 51.55 78.425) (width 1.016) (layer "B.Cu") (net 1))
 (segment (start 229.33 103.82) (end 231.4 103.82) (width 1.016) (layer "B.Cu") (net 1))
 (segment (start 231.42 78.43) (end 231.425 78.425) (width 1.016) (layer "B.Cu") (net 1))
 (segment (start 231.42 103.84) (end 231.42 78.43) (width 1.016) (layer "B.Cu") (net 1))
 (segment (start 231.425 78.425) (end 229.35 78.425) (width 1.016) (layer "B.Cu") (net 1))
 (segment (start 51.53 103.82) (end 229.33 103.82) (width 1.016) (layer "B.Cu") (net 1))
 (segment (start 49.595 93.655) (end 51.515 93.655) (width 1.016) (layer "F.Cu") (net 3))
 (segment (start 231.255 93.655) (end 229.34 93.655) (width 1.016) (layer "F.Cu") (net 3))
 (segment (start 49.56 93.62) (end 49.595 93.655) (width 1.016) (layer "F.Cu") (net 3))
 (segment (start 51.535 68.26) (end 229.36 68.26) (width 1.016) (layer "F.Cu") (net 3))
 (segment (start 51.535 68.26) (end 49.57 68.26) (width 1.016) (layer "F.Cu") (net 3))
 (segment (start 231.38 68.32) (end 231.38 93.53) (width 1.016) (layer "F.Cu") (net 3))
 (segment (start 49.57 68.26) (end 49.56 68.27) (width 1.016) (layer "F.Cu") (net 3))
 (segment (start 51.515 93.655) (end 229.34 93.655) (width 1.016) (layer "F.Cu") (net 3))
 (segment (start 231.38 93.53) (end 231.255 93.655) (width 1.016) (layer "F.Cu") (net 3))
 (segment (start 231.32 68.26) (end 231.38 68.32) (width 1.016) (layer "F.Cu") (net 3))
 (segment (start 153.115 93.655) (end 153.115 86.425) (width 1.016) (layer "F.Cu") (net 3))
 (segment (start 153.115 86.425) (end 151.475 84.785) (width 1.016) (layer "F.Cu") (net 3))
 (segment (start 229.36 68.26) (end 231.32 68.26) (width 1.016) (layer "F.Cu") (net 3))
 (segment (start 49.56 68.27) (end 49.56 93.62) (width 1.016) (layer "F.Cu") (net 3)))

